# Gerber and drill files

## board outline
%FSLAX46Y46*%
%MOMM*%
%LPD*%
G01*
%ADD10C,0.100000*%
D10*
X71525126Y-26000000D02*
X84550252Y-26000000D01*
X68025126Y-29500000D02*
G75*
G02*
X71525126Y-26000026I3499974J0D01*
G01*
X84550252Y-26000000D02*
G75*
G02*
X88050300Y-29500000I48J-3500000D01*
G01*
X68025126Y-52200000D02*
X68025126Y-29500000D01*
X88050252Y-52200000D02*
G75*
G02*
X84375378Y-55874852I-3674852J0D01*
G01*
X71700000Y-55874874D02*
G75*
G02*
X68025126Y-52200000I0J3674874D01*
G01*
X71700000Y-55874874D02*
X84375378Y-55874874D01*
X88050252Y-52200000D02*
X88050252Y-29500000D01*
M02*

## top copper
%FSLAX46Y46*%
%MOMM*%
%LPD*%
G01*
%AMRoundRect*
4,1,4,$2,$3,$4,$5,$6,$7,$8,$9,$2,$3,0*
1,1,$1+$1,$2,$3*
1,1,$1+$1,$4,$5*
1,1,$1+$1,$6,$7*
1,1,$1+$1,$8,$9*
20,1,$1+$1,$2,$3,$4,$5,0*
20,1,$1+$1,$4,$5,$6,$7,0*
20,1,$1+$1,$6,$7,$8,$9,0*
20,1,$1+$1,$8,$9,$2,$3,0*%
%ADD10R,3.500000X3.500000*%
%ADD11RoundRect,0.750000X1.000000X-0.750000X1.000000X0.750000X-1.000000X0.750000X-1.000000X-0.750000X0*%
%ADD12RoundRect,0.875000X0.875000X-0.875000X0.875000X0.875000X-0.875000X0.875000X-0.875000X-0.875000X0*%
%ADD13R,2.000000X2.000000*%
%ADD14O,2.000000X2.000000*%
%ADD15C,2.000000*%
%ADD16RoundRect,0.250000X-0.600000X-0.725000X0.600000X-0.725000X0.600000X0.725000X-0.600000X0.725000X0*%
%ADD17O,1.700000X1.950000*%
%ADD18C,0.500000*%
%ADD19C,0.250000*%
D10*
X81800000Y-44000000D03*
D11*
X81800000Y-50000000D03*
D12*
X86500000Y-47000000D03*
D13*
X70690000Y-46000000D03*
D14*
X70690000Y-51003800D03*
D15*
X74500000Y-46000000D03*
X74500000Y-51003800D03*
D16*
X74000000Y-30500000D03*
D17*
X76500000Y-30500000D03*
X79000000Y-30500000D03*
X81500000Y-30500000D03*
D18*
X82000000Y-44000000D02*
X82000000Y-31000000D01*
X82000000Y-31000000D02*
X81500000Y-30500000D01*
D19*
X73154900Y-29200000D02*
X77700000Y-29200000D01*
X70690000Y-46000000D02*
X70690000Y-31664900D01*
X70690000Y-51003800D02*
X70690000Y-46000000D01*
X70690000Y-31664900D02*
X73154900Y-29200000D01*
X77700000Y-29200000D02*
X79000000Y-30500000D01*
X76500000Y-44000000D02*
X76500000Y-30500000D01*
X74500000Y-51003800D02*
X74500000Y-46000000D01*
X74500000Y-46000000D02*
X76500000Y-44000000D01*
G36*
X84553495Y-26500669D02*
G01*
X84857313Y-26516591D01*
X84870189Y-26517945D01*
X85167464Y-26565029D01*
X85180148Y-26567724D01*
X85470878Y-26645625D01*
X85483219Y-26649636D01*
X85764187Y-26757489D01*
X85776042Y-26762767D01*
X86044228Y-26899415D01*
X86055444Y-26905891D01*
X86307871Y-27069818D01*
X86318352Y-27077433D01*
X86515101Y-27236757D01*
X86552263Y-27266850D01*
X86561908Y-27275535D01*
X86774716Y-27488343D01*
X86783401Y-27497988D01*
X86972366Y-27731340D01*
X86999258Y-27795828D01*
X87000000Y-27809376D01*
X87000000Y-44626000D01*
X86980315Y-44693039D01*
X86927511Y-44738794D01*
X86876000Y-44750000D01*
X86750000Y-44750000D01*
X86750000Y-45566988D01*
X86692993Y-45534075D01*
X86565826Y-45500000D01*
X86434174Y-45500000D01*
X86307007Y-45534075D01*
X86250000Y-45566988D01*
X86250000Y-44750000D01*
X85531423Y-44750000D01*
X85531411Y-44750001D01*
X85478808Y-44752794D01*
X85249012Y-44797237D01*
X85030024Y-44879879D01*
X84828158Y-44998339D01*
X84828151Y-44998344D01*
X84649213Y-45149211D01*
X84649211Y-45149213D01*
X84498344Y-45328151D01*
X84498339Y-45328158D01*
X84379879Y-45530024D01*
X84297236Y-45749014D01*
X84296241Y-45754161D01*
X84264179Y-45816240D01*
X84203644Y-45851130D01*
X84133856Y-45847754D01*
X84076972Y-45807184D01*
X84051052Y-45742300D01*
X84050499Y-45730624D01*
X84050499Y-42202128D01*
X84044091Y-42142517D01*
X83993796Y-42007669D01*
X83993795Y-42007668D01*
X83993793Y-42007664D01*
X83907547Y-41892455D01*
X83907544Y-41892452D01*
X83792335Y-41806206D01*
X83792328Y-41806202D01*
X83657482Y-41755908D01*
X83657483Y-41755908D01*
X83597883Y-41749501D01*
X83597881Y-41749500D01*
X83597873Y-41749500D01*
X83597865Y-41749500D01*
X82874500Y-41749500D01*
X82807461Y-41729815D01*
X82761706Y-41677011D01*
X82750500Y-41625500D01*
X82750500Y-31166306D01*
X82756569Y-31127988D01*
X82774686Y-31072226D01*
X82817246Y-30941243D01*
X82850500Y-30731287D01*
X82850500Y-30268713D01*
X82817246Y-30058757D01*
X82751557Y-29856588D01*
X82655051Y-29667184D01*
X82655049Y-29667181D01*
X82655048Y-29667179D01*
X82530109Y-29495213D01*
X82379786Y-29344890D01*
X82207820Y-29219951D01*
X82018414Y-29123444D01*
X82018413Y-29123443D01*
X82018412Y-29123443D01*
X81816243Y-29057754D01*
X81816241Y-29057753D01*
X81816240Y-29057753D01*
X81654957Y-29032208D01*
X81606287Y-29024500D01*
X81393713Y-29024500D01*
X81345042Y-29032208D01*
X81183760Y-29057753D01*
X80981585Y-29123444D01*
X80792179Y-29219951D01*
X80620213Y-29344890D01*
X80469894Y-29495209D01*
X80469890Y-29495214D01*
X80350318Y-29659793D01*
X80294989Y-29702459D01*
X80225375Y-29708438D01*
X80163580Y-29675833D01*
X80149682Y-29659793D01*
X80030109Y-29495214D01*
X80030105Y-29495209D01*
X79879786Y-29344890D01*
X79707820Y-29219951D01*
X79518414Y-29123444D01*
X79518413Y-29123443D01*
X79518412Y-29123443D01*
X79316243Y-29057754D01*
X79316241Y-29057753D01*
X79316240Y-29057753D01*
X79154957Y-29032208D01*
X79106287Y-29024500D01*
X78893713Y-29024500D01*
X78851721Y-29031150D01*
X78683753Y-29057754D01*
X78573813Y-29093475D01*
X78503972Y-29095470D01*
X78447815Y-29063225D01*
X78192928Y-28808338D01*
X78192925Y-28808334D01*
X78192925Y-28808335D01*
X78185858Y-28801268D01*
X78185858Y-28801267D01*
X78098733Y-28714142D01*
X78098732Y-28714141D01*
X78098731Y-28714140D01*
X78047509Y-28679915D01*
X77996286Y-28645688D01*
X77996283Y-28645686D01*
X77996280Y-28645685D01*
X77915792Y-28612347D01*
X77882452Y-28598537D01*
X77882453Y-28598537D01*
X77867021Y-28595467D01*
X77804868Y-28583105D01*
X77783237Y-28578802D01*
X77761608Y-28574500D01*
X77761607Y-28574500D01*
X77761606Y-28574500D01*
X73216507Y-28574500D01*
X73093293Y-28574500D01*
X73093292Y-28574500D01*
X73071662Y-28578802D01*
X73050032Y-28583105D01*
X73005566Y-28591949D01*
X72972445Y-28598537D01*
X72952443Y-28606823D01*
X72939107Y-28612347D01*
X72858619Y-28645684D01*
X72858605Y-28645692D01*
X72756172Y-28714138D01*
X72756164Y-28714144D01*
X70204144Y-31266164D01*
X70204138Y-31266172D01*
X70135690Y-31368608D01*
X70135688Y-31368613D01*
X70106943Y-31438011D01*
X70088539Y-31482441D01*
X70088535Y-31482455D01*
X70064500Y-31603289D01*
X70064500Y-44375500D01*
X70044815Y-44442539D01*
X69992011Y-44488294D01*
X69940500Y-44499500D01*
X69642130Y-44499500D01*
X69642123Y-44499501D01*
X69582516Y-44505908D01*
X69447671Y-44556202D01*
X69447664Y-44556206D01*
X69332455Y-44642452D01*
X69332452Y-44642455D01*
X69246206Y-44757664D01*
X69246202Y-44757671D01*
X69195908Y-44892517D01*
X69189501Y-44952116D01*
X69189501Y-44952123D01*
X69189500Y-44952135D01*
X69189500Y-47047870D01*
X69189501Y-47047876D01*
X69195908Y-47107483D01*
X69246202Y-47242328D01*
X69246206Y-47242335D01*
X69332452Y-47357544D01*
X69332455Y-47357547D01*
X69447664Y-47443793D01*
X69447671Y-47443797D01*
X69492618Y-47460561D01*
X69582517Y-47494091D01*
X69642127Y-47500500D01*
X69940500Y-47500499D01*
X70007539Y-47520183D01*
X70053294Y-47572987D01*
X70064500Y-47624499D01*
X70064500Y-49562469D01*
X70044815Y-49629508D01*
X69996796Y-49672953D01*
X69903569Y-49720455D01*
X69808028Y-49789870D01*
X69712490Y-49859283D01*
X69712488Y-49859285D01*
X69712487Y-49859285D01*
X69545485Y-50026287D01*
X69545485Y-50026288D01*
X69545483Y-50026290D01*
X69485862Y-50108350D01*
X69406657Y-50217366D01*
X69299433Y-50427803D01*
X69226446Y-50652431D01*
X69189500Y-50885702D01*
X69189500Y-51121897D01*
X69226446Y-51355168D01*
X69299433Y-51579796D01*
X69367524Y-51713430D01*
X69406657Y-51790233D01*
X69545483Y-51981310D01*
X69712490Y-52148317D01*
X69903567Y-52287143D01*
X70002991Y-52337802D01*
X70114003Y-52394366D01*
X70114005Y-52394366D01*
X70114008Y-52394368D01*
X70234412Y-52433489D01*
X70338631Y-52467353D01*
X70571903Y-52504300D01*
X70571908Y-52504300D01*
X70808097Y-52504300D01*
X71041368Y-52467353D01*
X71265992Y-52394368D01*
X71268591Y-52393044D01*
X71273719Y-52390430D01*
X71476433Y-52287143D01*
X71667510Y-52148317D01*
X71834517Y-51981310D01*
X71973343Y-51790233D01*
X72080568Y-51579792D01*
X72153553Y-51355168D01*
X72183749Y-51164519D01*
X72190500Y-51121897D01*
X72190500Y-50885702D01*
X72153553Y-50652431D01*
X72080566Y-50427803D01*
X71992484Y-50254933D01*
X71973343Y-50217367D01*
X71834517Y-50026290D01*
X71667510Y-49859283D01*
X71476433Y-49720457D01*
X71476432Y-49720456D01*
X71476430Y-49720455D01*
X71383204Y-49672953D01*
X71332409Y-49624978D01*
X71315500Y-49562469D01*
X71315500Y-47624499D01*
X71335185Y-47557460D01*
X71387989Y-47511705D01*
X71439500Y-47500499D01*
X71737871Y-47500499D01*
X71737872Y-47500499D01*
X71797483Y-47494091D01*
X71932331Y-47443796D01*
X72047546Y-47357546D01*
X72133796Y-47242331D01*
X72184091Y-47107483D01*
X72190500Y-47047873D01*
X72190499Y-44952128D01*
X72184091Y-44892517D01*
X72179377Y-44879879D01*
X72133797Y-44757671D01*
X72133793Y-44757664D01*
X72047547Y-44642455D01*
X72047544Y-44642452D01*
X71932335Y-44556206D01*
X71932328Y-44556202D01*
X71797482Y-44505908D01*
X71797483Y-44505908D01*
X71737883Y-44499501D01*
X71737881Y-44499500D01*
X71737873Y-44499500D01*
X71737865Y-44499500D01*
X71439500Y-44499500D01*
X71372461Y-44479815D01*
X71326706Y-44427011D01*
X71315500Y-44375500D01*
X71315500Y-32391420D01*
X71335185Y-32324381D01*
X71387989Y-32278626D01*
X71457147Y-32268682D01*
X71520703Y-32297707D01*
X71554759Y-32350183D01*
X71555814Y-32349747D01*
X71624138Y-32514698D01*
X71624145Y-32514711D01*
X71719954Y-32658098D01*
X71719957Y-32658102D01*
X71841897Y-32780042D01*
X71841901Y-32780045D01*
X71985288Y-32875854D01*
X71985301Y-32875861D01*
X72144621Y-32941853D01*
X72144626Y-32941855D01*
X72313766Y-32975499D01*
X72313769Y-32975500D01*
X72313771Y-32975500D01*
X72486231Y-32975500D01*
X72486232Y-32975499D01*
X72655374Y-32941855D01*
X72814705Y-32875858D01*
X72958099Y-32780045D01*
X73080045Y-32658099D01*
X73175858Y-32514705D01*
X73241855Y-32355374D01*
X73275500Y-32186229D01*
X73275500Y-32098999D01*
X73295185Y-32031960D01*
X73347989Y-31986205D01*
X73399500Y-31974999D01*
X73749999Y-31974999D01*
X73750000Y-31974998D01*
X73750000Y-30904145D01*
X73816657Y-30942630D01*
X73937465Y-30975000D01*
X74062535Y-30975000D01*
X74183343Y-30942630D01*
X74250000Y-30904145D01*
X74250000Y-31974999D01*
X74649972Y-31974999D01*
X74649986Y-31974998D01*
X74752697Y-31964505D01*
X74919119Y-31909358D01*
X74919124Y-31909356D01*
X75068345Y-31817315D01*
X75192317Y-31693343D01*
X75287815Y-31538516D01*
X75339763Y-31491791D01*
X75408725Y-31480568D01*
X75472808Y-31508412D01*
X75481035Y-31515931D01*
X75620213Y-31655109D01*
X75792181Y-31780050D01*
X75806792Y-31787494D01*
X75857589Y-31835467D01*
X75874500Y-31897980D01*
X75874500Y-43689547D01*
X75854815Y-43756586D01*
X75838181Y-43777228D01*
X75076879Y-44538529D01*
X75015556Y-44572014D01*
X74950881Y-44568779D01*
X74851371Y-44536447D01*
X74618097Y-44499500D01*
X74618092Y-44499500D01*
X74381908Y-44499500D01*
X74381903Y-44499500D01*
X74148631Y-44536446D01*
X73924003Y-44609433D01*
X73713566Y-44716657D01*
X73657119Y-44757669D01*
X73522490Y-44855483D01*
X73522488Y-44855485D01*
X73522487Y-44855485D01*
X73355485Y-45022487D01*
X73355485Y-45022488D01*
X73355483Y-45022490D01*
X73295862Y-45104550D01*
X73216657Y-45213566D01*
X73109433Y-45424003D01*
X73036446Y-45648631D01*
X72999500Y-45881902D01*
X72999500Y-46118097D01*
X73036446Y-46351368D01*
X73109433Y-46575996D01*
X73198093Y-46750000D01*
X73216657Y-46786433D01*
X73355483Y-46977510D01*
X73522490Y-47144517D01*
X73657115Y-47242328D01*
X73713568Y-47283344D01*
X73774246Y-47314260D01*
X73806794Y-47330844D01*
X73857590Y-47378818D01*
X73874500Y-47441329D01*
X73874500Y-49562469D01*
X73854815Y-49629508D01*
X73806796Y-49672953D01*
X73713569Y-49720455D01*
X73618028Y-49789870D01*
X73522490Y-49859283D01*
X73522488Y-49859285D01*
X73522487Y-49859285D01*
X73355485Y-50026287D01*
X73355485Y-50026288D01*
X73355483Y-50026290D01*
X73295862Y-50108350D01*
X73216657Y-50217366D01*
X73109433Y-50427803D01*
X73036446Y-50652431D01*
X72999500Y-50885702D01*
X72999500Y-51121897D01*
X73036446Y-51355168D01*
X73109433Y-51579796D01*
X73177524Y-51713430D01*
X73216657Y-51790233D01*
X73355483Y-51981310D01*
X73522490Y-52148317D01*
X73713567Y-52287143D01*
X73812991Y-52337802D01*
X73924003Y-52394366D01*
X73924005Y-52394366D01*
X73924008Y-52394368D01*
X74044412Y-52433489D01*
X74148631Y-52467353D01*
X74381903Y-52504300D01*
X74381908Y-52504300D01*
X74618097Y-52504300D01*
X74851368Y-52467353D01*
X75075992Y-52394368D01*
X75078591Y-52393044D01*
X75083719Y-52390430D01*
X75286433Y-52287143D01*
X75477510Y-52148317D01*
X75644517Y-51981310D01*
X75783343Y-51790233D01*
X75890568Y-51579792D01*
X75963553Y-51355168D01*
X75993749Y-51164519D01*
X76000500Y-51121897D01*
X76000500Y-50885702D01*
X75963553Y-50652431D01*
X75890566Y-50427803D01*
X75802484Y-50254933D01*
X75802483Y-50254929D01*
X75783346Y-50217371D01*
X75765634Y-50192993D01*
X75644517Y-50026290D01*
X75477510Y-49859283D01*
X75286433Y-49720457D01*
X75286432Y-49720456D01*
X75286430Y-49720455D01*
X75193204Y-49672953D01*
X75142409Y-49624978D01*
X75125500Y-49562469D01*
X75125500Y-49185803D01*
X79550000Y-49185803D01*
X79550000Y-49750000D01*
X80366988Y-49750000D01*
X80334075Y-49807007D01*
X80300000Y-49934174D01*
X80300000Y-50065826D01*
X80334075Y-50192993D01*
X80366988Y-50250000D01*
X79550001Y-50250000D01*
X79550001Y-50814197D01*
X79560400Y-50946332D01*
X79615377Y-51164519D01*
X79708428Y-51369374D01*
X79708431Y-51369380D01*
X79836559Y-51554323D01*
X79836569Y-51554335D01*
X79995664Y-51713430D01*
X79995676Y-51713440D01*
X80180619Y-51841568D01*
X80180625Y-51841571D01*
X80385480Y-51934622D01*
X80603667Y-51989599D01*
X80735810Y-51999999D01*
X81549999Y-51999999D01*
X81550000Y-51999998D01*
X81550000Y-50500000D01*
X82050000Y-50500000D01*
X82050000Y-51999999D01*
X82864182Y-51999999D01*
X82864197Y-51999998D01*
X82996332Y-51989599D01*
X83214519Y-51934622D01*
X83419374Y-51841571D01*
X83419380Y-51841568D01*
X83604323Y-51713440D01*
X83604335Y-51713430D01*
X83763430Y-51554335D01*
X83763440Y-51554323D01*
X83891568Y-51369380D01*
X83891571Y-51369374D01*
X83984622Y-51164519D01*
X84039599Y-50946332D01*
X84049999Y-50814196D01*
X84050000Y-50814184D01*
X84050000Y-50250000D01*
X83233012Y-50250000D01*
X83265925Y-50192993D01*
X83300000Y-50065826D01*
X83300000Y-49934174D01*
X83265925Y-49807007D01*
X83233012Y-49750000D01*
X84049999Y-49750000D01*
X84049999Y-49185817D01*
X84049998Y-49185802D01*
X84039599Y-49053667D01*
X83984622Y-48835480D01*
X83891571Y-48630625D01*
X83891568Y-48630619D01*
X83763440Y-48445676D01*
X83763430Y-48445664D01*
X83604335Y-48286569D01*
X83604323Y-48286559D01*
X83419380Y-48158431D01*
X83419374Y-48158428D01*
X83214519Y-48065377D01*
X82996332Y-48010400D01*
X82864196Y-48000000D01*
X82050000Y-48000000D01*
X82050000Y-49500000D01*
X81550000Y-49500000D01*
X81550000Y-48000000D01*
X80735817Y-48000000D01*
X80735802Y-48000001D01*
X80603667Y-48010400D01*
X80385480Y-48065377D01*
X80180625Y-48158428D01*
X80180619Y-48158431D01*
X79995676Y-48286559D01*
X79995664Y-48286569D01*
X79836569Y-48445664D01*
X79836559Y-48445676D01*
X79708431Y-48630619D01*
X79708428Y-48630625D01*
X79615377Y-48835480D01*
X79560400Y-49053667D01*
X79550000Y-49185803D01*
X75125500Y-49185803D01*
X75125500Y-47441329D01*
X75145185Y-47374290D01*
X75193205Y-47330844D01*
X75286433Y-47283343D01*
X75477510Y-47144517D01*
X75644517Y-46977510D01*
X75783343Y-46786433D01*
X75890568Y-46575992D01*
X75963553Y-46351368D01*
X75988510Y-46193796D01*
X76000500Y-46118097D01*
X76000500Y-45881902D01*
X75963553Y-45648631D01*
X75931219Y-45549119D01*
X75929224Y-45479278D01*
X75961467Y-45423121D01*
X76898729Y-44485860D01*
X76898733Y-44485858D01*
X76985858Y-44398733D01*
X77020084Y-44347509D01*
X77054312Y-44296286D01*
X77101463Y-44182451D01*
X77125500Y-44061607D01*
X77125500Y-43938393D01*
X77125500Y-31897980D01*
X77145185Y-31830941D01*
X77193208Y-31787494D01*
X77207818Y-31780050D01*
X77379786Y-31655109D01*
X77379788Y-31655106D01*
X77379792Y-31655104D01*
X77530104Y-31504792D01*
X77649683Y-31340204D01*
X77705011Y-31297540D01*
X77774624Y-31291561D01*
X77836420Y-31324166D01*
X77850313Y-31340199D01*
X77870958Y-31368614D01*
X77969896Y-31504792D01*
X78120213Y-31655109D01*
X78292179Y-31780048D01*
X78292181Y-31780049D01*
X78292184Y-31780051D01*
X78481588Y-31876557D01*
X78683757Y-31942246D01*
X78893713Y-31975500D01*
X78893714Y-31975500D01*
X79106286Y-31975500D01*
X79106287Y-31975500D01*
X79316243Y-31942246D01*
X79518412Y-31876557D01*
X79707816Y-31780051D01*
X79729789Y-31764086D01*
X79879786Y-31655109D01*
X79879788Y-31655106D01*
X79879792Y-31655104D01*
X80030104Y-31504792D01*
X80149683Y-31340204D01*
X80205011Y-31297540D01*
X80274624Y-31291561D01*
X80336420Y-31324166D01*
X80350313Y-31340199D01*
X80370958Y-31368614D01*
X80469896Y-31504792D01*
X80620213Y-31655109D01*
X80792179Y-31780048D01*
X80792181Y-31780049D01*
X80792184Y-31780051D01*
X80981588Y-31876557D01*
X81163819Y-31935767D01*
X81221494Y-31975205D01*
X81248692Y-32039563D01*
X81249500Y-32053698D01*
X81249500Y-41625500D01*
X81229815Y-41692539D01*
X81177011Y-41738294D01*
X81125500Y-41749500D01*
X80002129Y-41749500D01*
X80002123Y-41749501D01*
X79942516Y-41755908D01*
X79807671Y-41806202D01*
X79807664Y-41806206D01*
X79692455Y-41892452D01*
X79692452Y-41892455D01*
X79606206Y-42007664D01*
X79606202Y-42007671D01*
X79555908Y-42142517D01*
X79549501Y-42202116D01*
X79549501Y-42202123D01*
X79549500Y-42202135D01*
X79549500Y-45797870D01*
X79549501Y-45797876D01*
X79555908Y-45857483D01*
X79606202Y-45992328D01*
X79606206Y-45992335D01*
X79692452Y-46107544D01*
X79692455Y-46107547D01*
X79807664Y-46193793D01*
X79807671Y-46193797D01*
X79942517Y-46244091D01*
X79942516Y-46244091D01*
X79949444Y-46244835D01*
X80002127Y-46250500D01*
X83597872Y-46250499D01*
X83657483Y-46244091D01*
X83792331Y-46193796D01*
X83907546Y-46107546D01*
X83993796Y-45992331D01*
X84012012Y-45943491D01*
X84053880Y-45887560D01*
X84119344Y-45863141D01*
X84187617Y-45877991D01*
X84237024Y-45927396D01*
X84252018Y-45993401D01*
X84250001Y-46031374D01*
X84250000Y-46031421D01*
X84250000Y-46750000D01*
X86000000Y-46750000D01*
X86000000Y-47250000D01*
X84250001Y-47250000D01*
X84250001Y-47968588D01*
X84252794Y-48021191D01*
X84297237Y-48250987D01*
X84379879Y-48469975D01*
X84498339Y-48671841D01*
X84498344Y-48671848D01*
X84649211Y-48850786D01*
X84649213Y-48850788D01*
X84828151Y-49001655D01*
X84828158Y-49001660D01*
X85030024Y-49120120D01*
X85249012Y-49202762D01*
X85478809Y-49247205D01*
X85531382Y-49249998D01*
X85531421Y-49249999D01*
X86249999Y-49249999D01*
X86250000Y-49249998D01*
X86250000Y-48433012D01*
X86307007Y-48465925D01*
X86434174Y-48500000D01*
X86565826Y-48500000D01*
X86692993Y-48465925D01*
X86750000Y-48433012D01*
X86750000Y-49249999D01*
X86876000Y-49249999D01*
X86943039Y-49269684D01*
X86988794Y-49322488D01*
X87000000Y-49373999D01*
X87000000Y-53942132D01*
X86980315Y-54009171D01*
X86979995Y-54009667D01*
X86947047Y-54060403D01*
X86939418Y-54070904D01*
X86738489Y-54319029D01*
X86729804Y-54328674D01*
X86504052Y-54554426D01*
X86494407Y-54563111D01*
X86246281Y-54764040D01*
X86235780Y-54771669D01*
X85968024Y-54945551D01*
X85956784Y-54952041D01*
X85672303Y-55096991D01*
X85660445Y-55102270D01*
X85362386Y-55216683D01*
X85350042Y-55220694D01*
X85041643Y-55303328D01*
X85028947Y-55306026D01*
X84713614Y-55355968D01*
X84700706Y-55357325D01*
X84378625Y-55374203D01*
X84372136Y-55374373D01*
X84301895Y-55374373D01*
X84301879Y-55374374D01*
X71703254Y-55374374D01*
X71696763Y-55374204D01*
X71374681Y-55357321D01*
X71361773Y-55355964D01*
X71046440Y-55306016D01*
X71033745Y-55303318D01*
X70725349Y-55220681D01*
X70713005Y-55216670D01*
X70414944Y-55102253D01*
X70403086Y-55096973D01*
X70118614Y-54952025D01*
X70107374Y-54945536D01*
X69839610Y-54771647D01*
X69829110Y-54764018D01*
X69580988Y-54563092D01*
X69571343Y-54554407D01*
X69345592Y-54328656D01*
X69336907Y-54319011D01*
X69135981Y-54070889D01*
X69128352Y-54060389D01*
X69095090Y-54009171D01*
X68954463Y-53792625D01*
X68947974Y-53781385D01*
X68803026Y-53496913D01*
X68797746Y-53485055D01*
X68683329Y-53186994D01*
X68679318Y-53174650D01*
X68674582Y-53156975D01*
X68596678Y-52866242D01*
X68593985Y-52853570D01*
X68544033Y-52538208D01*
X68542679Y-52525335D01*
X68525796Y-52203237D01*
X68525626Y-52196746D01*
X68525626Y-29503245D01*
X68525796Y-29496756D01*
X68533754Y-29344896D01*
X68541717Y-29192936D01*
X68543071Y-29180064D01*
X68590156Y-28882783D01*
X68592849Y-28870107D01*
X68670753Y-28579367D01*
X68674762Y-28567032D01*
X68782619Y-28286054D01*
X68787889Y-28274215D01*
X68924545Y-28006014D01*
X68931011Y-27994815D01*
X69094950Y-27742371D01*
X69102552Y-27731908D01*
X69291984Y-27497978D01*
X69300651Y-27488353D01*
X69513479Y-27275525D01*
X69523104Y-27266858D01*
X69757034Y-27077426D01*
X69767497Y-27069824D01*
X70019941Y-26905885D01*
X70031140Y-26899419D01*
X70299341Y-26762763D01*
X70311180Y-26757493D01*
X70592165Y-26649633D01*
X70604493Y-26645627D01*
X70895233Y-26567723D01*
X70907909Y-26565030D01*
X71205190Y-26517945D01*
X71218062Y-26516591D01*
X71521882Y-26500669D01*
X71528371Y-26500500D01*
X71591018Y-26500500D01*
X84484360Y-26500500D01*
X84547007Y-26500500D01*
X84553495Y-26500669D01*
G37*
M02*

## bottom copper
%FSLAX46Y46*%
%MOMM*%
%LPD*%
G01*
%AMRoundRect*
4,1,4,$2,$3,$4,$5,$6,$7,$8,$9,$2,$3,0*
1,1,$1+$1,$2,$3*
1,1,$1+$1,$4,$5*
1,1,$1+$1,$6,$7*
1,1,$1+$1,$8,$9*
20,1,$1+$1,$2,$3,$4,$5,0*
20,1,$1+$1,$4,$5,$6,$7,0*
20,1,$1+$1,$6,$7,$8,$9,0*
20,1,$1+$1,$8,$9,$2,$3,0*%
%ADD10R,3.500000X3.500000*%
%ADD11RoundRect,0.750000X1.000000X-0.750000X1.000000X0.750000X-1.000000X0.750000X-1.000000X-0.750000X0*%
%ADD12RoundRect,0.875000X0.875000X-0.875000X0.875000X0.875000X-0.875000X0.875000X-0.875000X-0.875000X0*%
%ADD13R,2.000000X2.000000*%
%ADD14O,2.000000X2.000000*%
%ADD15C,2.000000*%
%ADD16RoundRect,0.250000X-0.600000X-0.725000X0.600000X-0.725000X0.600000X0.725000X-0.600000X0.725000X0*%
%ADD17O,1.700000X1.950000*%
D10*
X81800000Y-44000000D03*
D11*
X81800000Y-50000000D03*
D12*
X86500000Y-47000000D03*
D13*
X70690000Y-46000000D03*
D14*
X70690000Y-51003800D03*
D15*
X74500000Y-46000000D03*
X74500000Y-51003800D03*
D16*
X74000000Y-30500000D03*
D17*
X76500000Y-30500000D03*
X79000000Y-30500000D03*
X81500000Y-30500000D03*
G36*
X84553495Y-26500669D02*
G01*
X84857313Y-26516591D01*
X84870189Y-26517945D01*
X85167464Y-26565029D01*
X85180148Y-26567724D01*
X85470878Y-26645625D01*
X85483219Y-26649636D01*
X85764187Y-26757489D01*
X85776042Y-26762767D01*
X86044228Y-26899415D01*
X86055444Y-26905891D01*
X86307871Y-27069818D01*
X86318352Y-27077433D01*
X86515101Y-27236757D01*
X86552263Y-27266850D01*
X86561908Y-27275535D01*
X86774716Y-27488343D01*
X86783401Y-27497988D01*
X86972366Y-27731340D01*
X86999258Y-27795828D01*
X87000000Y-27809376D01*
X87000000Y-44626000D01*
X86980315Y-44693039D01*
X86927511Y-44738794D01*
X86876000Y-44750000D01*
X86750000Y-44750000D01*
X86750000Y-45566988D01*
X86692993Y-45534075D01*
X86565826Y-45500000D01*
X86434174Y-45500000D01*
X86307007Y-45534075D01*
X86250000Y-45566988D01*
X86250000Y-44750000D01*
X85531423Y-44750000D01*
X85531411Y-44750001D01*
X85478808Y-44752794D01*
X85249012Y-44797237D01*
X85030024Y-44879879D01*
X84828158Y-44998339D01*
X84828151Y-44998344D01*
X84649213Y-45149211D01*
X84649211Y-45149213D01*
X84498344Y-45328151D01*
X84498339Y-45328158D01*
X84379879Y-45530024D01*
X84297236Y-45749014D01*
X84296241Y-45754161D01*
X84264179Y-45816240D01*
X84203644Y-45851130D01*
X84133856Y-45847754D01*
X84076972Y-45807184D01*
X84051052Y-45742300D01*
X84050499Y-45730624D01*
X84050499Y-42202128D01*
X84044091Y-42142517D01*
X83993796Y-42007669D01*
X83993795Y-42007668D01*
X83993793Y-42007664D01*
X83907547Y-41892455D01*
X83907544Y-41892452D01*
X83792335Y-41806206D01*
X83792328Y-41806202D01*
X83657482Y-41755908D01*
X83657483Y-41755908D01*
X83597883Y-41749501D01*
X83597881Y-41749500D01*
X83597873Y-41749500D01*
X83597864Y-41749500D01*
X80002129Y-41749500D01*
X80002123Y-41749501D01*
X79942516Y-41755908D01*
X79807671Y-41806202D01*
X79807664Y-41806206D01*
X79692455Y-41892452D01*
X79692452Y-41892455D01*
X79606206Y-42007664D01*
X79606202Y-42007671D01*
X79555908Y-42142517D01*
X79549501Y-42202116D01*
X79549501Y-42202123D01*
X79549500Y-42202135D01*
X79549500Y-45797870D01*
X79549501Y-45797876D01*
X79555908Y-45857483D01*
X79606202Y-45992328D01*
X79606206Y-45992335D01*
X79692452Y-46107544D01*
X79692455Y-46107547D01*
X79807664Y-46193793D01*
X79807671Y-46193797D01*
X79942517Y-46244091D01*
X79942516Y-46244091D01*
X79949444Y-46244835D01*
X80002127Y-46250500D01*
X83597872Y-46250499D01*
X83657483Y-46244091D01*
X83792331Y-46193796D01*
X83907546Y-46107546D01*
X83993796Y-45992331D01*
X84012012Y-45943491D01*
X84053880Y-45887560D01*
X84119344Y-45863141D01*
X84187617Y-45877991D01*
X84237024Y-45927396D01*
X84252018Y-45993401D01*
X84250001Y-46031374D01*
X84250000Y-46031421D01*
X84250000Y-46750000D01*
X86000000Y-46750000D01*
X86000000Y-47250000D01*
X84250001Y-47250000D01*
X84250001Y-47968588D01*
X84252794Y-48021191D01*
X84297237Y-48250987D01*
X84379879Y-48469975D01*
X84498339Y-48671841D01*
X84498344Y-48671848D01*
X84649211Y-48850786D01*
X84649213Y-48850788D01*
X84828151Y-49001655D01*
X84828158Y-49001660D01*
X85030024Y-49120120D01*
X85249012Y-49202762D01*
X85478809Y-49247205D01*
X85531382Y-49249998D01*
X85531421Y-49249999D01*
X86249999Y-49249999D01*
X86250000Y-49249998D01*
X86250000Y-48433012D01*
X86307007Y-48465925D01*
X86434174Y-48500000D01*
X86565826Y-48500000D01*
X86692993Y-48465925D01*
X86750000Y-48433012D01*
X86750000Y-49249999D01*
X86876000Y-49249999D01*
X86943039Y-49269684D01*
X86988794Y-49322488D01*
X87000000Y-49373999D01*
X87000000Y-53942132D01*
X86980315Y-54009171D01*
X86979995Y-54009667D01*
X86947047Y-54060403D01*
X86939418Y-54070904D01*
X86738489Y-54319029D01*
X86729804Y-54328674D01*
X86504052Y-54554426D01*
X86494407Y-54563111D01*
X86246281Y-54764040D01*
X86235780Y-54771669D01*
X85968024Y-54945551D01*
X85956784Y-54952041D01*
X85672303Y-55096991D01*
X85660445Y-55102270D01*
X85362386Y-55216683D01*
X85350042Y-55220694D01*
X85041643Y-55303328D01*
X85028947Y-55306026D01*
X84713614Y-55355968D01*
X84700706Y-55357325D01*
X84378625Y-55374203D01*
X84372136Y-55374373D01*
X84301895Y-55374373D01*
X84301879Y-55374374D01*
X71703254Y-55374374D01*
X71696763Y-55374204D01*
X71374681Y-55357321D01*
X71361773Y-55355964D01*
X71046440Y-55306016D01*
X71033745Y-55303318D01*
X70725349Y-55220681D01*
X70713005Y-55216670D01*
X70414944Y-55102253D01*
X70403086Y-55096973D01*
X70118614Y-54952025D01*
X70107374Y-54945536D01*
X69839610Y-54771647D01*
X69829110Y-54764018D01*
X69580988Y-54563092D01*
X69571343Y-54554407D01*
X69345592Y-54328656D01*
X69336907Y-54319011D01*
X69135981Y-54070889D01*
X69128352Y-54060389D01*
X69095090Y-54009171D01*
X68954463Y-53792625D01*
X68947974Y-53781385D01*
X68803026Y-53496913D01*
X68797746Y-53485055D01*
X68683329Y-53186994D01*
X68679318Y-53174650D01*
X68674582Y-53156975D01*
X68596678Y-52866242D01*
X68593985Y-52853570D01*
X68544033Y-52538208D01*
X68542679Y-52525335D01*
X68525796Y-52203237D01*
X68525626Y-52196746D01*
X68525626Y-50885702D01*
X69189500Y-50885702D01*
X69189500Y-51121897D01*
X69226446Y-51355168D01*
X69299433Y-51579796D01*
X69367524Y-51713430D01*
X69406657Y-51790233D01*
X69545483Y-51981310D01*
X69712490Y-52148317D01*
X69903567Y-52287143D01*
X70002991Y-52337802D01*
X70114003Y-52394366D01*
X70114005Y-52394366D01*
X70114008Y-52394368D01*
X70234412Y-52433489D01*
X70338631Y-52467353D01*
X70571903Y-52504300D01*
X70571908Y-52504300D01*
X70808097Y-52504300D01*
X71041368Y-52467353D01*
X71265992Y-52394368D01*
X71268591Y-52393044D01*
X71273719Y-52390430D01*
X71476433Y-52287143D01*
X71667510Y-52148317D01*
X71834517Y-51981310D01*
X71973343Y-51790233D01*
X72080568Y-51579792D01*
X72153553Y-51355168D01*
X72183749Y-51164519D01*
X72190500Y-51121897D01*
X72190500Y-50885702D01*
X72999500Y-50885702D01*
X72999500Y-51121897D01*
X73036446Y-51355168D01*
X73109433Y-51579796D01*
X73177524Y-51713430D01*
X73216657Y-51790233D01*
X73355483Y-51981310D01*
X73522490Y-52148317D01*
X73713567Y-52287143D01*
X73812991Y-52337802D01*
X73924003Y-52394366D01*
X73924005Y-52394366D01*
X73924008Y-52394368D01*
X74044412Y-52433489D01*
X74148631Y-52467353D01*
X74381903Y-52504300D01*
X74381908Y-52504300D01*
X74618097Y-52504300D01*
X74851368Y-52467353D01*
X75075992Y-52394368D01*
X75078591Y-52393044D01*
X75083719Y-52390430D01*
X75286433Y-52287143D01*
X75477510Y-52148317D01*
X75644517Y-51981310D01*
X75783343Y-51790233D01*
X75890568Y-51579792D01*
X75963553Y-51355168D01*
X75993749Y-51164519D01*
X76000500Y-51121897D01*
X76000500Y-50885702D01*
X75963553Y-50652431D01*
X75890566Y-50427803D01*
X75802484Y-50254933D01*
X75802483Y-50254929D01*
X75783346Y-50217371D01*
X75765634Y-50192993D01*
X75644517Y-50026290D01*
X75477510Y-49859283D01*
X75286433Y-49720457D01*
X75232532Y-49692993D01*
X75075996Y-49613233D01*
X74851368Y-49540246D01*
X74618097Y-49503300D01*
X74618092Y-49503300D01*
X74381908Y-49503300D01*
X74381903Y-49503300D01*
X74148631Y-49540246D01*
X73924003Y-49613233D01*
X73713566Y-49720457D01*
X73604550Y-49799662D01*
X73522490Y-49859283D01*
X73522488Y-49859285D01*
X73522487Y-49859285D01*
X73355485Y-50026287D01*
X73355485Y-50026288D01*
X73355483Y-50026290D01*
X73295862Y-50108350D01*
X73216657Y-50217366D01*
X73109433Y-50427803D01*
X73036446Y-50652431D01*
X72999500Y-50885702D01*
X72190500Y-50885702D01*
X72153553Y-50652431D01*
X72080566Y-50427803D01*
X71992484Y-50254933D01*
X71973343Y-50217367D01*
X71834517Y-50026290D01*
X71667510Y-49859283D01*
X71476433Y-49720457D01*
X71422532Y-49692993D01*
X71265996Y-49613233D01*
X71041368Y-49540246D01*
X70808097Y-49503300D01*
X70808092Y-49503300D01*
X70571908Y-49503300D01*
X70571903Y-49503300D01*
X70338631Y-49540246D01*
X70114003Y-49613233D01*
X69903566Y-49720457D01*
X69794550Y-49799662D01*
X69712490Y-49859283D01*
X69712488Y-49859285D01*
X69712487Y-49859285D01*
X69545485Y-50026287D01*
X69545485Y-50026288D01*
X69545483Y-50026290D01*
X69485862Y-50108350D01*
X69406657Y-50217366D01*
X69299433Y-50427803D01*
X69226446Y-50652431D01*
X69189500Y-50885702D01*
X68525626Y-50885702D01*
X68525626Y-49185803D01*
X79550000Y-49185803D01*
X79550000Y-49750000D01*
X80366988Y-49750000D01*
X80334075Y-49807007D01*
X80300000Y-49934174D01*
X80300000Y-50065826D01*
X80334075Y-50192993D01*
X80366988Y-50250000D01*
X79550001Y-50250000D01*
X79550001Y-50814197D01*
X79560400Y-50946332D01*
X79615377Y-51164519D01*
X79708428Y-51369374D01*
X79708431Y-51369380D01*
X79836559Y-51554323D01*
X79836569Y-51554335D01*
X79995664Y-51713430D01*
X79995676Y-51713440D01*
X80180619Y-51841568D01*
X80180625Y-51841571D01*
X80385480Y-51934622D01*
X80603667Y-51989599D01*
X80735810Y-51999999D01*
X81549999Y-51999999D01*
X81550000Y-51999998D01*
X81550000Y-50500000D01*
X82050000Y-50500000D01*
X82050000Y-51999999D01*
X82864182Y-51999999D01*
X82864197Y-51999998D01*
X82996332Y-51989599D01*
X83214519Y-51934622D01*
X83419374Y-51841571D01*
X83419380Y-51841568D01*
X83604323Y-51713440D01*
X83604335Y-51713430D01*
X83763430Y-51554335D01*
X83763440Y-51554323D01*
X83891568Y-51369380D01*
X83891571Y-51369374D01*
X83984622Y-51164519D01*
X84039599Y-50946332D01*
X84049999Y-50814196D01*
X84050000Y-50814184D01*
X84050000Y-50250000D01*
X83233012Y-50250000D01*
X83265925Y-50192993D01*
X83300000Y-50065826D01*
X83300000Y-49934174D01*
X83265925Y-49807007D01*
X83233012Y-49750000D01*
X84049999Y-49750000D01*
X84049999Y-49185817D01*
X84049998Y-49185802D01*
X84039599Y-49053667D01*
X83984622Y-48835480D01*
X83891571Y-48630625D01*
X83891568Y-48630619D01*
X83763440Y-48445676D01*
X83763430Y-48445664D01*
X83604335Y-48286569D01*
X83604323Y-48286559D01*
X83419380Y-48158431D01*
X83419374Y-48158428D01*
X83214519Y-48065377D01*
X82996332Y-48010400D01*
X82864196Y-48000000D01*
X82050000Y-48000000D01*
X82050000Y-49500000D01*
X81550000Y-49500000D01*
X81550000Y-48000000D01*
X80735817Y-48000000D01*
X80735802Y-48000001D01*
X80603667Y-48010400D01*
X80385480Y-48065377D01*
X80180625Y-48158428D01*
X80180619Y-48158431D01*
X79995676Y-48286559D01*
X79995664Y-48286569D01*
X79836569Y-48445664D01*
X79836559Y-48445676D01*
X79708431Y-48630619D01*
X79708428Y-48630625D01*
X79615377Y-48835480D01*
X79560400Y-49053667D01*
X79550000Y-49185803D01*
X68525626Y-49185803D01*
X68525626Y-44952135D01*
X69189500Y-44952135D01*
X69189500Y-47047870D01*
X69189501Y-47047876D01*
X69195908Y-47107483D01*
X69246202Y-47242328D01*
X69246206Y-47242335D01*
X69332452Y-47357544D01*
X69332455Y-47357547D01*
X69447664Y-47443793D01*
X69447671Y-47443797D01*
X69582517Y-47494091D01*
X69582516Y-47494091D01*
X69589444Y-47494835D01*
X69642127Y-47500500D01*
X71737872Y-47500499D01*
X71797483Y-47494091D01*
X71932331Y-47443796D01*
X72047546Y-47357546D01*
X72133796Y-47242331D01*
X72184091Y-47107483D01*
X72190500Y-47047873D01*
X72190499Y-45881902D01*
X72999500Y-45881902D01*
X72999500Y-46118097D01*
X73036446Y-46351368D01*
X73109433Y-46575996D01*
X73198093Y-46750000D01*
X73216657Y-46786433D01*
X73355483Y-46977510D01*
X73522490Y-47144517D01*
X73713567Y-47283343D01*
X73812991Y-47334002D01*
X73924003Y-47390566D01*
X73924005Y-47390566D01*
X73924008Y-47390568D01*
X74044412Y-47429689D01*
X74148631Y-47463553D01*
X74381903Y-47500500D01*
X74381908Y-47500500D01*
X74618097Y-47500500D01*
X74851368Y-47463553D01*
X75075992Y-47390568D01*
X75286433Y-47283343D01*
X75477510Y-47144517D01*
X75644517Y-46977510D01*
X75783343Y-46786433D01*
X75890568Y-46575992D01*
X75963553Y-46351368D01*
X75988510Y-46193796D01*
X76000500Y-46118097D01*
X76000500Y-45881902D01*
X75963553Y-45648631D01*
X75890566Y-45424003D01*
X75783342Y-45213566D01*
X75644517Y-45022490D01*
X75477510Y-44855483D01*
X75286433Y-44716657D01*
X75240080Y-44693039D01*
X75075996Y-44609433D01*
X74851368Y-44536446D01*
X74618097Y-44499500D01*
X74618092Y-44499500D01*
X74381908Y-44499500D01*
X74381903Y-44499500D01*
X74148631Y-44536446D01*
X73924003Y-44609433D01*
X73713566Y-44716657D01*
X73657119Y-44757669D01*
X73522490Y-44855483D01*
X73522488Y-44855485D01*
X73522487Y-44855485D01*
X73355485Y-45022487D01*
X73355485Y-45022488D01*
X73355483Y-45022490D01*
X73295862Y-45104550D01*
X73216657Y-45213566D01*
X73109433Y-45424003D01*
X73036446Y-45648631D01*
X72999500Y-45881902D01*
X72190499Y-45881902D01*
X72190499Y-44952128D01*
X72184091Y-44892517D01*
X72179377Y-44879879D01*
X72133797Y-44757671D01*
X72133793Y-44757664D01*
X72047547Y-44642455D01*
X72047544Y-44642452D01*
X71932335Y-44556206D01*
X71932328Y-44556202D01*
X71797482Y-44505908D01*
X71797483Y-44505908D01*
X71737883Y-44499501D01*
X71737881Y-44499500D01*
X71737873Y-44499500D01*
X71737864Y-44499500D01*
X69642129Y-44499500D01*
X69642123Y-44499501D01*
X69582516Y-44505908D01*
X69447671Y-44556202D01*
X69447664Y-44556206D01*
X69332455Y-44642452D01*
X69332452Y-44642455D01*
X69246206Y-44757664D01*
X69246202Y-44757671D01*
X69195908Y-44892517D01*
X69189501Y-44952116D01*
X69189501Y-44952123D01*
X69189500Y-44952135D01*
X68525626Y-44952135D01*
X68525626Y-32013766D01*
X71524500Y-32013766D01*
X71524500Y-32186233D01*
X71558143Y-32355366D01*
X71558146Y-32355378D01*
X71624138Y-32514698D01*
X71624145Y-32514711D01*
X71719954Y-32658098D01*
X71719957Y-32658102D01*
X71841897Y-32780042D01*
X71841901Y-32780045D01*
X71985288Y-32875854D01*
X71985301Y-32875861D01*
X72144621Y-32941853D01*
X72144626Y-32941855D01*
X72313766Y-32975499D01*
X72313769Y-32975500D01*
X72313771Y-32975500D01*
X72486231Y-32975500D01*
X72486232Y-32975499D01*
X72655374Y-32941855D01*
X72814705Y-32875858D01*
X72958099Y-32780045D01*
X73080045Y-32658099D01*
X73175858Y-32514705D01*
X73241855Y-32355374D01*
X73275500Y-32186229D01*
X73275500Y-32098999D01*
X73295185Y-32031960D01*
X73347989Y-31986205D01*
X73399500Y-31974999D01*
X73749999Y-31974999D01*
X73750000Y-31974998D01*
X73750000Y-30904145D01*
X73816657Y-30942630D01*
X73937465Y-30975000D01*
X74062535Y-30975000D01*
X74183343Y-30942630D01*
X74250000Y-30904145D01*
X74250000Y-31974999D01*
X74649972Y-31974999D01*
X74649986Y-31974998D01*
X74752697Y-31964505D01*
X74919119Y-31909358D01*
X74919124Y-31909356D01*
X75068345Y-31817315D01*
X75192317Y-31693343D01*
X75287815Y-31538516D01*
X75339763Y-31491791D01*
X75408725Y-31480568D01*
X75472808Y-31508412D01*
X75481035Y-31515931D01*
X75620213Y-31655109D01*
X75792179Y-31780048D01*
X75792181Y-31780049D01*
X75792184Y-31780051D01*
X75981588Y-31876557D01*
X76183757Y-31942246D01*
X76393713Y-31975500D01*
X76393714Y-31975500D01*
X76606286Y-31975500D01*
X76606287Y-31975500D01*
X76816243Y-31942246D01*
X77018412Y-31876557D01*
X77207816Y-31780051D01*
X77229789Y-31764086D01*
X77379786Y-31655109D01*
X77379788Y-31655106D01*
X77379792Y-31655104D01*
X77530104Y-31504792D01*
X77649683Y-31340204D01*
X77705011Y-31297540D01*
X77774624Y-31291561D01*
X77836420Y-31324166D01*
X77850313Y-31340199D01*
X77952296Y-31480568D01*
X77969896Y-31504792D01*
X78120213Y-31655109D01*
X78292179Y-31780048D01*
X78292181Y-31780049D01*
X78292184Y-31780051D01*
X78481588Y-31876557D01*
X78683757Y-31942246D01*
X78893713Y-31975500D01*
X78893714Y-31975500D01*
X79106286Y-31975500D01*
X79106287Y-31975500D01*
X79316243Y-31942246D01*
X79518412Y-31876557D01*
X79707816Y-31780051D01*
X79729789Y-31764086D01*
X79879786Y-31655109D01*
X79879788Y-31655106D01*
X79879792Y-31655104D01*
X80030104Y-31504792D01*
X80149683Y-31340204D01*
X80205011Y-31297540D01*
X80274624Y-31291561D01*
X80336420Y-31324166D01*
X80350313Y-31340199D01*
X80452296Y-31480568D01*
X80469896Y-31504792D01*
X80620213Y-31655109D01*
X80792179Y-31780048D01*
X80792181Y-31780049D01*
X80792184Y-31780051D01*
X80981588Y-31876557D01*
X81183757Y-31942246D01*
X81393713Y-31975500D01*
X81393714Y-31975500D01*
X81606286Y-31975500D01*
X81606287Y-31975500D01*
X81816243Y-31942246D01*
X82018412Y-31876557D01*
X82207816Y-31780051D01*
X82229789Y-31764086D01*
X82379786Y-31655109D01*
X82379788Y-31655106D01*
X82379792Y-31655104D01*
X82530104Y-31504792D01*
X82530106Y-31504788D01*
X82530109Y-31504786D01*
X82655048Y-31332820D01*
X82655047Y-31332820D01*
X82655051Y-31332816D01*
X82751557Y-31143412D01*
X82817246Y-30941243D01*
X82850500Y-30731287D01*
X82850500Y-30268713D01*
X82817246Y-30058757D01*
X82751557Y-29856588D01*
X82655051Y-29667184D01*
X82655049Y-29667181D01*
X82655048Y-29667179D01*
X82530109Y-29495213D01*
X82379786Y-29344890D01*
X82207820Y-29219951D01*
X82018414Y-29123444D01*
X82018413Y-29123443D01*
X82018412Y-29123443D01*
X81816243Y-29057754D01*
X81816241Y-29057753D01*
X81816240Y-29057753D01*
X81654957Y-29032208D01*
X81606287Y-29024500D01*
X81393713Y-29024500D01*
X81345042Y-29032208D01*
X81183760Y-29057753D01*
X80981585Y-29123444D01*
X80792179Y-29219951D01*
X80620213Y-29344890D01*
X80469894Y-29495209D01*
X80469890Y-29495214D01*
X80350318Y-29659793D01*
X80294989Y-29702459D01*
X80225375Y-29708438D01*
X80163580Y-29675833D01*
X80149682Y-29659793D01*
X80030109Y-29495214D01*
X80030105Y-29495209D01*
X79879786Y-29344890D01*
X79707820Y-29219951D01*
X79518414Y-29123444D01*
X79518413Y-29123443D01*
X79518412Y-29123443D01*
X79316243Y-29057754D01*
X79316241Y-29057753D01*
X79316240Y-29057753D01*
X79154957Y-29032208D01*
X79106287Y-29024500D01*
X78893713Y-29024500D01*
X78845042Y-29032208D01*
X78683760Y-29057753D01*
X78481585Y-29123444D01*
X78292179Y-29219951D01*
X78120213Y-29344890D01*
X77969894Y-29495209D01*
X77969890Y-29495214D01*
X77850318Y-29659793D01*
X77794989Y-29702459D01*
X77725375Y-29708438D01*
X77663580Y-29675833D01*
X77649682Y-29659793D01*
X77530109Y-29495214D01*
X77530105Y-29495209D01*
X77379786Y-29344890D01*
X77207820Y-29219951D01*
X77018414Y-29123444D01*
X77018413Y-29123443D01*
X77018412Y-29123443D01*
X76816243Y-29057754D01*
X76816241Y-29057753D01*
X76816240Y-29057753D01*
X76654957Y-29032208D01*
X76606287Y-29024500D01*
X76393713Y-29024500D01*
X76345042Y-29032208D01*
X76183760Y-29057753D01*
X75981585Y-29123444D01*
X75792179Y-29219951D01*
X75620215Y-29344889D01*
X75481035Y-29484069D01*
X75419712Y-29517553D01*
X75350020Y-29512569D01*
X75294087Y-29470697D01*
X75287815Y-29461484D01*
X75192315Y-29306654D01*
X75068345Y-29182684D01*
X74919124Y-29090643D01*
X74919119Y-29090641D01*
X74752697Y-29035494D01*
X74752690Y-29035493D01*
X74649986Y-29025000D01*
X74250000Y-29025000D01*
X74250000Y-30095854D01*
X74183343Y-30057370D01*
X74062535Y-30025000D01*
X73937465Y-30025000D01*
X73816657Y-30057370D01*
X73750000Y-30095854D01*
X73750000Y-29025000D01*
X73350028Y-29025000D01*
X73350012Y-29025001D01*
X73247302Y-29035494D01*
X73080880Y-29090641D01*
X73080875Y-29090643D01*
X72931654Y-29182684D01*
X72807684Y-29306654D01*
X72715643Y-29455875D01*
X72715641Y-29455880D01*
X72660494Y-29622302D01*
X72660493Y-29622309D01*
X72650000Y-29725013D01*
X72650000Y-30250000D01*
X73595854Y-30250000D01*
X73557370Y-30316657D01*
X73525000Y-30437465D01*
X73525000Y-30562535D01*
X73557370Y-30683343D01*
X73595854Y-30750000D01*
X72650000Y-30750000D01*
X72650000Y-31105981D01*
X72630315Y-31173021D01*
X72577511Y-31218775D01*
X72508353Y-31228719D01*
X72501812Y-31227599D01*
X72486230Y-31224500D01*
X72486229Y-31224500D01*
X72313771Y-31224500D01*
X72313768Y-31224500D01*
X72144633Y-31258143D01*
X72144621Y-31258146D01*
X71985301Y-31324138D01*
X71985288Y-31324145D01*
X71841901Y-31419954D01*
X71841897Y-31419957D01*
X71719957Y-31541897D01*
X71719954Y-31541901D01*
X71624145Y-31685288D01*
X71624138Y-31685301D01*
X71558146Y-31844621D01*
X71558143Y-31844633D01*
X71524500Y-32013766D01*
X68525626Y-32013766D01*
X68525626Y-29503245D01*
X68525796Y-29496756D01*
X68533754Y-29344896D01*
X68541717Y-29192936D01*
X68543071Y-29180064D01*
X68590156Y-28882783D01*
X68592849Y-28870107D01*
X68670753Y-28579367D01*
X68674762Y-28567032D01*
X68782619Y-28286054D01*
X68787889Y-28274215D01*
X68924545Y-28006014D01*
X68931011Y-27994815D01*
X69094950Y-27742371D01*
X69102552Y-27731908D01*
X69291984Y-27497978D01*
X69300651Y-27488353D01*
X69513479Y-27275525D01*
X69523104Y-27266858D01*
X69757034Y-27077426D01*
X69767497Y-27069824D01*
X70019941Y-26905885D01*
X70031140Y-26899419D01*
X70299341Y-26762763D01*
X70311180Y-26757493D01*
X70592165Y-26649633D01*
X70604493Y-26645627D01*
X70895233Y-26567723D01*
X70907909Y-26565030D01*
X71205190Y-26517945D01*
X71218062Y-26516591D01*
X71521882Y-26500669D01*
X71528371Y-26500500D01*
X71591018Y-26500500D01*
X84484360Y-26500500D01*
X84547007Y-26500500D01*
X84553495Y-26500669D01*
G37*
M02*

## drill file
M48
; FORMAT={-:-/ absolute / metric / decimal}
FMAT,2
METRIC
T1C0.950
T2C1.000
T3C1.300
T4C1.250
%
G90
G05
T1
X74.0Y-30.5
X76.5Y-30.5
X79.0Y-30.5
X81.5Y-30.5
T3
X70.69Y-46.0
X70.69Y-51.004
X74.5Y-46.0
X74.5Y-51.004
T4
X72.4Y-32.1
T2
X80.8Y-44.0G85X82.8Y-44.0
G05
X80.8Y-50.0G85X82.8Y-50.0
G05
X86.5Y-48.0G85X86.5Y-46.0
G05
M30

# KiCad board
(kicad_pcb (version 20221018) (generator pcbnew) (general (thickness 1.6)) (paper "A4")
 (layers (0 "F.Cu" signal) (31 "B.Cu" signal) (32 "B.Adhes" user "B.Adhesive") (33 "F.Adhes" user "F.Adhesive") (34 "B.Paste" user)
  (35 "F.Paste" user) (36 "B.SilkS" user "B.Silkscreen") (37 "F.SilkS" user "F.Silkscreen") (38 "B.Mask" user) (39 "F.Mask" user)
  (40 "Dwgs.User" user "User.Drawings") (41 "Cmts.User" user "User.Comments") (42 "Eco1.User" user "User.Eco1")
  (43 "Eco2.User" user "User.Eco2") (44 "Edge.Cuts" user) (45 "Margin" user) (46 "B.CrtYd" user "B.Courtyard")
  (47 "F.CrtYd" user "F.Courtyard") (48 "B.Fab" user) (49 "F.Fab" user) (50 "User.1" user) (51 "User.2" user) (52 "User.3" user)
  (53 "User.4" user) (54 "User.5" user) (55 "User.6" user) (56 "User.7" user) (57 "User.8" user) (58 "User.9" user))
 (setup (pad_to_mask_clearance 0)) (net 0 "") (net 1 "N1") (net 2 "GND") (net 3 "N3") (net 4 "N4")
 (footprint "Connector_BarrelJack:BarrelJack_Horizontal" (layer "F.Cu") (at 81.8 44 90)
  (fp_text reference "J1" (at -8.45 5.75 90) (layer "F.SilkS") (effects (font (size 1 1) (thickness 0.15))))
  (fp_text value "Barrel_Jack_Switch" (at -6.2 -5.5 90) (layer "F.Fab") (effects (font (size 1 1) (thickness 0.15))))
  (pad "1" thru_hole rect (at 0 0 90) (size 3.5 3.5) (drill oval 1 3) (layers "*.Cu" "*.Mask") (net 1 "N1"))
  (pad "2" thru_hole roundrect (at -6 0 90) (size 3 3.5) (drill oval 1 3) (layers "*.Cu" "*.Mask") (roundrect_rratio 0.25) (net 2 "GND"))
  (pad "3" thru_hole roundrect (at -3 4.7 90) (size 3.5 3.5) (drill oval 3 1) (layers "*.Cu" "*.Mask") (roundrect_rratio 0.25) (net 2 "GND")))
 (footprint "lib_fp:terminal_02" (layer "F.Cu") (at 70.69 46)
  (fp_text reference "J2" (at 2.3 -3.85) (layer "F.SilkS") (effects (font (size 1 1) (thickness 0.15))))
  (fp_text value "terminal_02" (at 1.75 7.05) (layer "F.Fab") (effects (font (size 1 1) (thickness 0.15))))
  (pad "1" thru_hole rect (at 0 0) (size 2 2) (drill 1.3) (layers "*.Cu" "*.Mask") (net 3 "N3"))
  (pad "1" thru_hole oval (at 0 5.0038) (size 2 2) (drill 1.3) (layers "*.Cu" "*.Mask") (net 3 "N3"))
  (pad "2" thru_hole circle (at 3.81 0) (size 2 2) (drill 1.3) (layers "*.Cu" "*.Mask") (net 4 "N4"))
  (pad "2" thru_hole circle (at 3.81 5.0038) (size 2 2) (drill 1.3) (layers "*.Cu" "*.Mask") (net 4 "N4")))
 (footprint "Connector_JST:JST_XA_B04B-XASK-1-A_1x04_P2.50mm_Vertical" (layer "F.Cu") (at 74 30.5)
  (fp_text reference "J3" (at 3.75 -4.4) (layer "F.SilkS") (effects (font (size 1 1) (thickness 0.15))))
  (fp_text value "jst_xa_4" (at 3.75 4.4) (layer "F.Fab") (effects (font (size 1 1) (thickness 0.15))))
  (pad "" np_thru_hole circle (at -1.6 1.6) (size 1.25 1.25) (drill 1.25) (layers "*.Cu" "*.Mask"))
  (pad "1" thru_hole roundrect (at 0 0) (size 1.7 1.95) (drill 0.95) (layers "*.Cu" "*.Mask") (roundrect_rratio 0.1470588235) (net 2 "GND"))
  (pad "2" thru_hole oval (at 2.5 0) (size 1.7 1.95) (drill 0.95) (layers "*.Cu" "*.Mask") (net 4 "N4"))
  (pad "3" thru_hole oval (at 5 0) (size 1.7 1.95) (drill 0.95) (layers "*.Cu" "*.Mask") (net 3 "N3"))
  (pad "4" thru_hole oval (at 7.5 0) (size 1.7 1.95) (drill 0.95) (layers "*.Cu" "*.Mask") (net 1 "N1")))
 (gr_line (start 71.525126 26) (end 84.550252 26) (stroke (width 0.1) (type default)) (layer "Edge.Cuts"))
 (gr_arc (start 68.025126 29.5) (mid 69.050252 27.025126) (end 71.525126 26) (stroke (width 0.1) (type default)) (layer "Edge.Cuts"))
 (gr_arc (start 84.550252 26) (mid 87.025126 27.025126) (end 88.050252 29.5) (stroke (width 0.1) (type default)) (layer "Edge.Cuts"))
 (gr_line (start 68.025126 52.2) (end 68.025126 29.5) (stroke (width 0.1) (type default)) (layer "Edge.Cuts"))
 (gr_arc (start 88.050252 52.2) (mid 86.973912 54.798534) (end 84.375378 55.874874) (stroke (width 0.1) (type default)) (layer "Edge.Cuts"))
 (gr_arc (start 71.7 55.874874) (mid 69.101485 54.798515) (end 68.025126 52.2) (stroke (width 0.1) (type default)) (layer "Edge.Cuts"))
 (gr_line (start 71.7 55.874874) (end 84.375378 55.874874) (stroke (width 0.1) (type default)) (layer "Edge.Cuts"))
 (gr_line (start 88.050252 52.2) (end 88.050252 29.5) (stroke (width 0.1) (type default)) (layer "Edge.Cuts"))
 (segment (start 82 44) (end 82 31) (width 0.5) (layer "F.Cu") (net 1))
 (segment (start 82 31) (end 81.5 30.5) (width 0.5) (layer "F.Cu") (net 1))
 (segment (start 73.1549 29.2) (end 77.7 29.2) (width 0.25) (layer "F.Cu") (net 3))
 (segment (start 70.69 46) (end 70.69 31.6649) (width 0.25) (layer "F.Cu") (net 3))
 (segment (start 70.69 51.0038) (end 70.69 46) (width 0.25) (layer "F.Cu") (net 3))
 (segment (start 70.69 31.6649) (end 73.1549 29.2) (width 0.25) (layer "F.Cu") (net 3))
 (segment (start 77.7 29.2) (end 79 30.5) (width 0.25) (layer "F.Cu") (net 3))
 (segment (start 76.5 44) (end 76.5 30.5) (width 0.25) (layer "F.Cu") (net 4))
 (segment (start 74.5 51.0038) (end 74.5 46) (width 0.25) (layer "F.Cu") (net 4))
 (segment (start 74.5 46) (end 76.5 44) (width 0.25) (layer "F.Cu") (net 4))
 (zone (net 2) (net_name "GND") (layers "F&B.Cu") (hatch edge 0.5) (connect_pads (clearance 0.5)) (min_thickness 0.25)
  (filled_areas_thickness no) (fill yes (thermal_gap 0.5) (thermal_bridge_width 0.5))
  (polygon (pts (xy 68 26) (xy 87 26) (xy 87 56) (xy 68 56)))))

